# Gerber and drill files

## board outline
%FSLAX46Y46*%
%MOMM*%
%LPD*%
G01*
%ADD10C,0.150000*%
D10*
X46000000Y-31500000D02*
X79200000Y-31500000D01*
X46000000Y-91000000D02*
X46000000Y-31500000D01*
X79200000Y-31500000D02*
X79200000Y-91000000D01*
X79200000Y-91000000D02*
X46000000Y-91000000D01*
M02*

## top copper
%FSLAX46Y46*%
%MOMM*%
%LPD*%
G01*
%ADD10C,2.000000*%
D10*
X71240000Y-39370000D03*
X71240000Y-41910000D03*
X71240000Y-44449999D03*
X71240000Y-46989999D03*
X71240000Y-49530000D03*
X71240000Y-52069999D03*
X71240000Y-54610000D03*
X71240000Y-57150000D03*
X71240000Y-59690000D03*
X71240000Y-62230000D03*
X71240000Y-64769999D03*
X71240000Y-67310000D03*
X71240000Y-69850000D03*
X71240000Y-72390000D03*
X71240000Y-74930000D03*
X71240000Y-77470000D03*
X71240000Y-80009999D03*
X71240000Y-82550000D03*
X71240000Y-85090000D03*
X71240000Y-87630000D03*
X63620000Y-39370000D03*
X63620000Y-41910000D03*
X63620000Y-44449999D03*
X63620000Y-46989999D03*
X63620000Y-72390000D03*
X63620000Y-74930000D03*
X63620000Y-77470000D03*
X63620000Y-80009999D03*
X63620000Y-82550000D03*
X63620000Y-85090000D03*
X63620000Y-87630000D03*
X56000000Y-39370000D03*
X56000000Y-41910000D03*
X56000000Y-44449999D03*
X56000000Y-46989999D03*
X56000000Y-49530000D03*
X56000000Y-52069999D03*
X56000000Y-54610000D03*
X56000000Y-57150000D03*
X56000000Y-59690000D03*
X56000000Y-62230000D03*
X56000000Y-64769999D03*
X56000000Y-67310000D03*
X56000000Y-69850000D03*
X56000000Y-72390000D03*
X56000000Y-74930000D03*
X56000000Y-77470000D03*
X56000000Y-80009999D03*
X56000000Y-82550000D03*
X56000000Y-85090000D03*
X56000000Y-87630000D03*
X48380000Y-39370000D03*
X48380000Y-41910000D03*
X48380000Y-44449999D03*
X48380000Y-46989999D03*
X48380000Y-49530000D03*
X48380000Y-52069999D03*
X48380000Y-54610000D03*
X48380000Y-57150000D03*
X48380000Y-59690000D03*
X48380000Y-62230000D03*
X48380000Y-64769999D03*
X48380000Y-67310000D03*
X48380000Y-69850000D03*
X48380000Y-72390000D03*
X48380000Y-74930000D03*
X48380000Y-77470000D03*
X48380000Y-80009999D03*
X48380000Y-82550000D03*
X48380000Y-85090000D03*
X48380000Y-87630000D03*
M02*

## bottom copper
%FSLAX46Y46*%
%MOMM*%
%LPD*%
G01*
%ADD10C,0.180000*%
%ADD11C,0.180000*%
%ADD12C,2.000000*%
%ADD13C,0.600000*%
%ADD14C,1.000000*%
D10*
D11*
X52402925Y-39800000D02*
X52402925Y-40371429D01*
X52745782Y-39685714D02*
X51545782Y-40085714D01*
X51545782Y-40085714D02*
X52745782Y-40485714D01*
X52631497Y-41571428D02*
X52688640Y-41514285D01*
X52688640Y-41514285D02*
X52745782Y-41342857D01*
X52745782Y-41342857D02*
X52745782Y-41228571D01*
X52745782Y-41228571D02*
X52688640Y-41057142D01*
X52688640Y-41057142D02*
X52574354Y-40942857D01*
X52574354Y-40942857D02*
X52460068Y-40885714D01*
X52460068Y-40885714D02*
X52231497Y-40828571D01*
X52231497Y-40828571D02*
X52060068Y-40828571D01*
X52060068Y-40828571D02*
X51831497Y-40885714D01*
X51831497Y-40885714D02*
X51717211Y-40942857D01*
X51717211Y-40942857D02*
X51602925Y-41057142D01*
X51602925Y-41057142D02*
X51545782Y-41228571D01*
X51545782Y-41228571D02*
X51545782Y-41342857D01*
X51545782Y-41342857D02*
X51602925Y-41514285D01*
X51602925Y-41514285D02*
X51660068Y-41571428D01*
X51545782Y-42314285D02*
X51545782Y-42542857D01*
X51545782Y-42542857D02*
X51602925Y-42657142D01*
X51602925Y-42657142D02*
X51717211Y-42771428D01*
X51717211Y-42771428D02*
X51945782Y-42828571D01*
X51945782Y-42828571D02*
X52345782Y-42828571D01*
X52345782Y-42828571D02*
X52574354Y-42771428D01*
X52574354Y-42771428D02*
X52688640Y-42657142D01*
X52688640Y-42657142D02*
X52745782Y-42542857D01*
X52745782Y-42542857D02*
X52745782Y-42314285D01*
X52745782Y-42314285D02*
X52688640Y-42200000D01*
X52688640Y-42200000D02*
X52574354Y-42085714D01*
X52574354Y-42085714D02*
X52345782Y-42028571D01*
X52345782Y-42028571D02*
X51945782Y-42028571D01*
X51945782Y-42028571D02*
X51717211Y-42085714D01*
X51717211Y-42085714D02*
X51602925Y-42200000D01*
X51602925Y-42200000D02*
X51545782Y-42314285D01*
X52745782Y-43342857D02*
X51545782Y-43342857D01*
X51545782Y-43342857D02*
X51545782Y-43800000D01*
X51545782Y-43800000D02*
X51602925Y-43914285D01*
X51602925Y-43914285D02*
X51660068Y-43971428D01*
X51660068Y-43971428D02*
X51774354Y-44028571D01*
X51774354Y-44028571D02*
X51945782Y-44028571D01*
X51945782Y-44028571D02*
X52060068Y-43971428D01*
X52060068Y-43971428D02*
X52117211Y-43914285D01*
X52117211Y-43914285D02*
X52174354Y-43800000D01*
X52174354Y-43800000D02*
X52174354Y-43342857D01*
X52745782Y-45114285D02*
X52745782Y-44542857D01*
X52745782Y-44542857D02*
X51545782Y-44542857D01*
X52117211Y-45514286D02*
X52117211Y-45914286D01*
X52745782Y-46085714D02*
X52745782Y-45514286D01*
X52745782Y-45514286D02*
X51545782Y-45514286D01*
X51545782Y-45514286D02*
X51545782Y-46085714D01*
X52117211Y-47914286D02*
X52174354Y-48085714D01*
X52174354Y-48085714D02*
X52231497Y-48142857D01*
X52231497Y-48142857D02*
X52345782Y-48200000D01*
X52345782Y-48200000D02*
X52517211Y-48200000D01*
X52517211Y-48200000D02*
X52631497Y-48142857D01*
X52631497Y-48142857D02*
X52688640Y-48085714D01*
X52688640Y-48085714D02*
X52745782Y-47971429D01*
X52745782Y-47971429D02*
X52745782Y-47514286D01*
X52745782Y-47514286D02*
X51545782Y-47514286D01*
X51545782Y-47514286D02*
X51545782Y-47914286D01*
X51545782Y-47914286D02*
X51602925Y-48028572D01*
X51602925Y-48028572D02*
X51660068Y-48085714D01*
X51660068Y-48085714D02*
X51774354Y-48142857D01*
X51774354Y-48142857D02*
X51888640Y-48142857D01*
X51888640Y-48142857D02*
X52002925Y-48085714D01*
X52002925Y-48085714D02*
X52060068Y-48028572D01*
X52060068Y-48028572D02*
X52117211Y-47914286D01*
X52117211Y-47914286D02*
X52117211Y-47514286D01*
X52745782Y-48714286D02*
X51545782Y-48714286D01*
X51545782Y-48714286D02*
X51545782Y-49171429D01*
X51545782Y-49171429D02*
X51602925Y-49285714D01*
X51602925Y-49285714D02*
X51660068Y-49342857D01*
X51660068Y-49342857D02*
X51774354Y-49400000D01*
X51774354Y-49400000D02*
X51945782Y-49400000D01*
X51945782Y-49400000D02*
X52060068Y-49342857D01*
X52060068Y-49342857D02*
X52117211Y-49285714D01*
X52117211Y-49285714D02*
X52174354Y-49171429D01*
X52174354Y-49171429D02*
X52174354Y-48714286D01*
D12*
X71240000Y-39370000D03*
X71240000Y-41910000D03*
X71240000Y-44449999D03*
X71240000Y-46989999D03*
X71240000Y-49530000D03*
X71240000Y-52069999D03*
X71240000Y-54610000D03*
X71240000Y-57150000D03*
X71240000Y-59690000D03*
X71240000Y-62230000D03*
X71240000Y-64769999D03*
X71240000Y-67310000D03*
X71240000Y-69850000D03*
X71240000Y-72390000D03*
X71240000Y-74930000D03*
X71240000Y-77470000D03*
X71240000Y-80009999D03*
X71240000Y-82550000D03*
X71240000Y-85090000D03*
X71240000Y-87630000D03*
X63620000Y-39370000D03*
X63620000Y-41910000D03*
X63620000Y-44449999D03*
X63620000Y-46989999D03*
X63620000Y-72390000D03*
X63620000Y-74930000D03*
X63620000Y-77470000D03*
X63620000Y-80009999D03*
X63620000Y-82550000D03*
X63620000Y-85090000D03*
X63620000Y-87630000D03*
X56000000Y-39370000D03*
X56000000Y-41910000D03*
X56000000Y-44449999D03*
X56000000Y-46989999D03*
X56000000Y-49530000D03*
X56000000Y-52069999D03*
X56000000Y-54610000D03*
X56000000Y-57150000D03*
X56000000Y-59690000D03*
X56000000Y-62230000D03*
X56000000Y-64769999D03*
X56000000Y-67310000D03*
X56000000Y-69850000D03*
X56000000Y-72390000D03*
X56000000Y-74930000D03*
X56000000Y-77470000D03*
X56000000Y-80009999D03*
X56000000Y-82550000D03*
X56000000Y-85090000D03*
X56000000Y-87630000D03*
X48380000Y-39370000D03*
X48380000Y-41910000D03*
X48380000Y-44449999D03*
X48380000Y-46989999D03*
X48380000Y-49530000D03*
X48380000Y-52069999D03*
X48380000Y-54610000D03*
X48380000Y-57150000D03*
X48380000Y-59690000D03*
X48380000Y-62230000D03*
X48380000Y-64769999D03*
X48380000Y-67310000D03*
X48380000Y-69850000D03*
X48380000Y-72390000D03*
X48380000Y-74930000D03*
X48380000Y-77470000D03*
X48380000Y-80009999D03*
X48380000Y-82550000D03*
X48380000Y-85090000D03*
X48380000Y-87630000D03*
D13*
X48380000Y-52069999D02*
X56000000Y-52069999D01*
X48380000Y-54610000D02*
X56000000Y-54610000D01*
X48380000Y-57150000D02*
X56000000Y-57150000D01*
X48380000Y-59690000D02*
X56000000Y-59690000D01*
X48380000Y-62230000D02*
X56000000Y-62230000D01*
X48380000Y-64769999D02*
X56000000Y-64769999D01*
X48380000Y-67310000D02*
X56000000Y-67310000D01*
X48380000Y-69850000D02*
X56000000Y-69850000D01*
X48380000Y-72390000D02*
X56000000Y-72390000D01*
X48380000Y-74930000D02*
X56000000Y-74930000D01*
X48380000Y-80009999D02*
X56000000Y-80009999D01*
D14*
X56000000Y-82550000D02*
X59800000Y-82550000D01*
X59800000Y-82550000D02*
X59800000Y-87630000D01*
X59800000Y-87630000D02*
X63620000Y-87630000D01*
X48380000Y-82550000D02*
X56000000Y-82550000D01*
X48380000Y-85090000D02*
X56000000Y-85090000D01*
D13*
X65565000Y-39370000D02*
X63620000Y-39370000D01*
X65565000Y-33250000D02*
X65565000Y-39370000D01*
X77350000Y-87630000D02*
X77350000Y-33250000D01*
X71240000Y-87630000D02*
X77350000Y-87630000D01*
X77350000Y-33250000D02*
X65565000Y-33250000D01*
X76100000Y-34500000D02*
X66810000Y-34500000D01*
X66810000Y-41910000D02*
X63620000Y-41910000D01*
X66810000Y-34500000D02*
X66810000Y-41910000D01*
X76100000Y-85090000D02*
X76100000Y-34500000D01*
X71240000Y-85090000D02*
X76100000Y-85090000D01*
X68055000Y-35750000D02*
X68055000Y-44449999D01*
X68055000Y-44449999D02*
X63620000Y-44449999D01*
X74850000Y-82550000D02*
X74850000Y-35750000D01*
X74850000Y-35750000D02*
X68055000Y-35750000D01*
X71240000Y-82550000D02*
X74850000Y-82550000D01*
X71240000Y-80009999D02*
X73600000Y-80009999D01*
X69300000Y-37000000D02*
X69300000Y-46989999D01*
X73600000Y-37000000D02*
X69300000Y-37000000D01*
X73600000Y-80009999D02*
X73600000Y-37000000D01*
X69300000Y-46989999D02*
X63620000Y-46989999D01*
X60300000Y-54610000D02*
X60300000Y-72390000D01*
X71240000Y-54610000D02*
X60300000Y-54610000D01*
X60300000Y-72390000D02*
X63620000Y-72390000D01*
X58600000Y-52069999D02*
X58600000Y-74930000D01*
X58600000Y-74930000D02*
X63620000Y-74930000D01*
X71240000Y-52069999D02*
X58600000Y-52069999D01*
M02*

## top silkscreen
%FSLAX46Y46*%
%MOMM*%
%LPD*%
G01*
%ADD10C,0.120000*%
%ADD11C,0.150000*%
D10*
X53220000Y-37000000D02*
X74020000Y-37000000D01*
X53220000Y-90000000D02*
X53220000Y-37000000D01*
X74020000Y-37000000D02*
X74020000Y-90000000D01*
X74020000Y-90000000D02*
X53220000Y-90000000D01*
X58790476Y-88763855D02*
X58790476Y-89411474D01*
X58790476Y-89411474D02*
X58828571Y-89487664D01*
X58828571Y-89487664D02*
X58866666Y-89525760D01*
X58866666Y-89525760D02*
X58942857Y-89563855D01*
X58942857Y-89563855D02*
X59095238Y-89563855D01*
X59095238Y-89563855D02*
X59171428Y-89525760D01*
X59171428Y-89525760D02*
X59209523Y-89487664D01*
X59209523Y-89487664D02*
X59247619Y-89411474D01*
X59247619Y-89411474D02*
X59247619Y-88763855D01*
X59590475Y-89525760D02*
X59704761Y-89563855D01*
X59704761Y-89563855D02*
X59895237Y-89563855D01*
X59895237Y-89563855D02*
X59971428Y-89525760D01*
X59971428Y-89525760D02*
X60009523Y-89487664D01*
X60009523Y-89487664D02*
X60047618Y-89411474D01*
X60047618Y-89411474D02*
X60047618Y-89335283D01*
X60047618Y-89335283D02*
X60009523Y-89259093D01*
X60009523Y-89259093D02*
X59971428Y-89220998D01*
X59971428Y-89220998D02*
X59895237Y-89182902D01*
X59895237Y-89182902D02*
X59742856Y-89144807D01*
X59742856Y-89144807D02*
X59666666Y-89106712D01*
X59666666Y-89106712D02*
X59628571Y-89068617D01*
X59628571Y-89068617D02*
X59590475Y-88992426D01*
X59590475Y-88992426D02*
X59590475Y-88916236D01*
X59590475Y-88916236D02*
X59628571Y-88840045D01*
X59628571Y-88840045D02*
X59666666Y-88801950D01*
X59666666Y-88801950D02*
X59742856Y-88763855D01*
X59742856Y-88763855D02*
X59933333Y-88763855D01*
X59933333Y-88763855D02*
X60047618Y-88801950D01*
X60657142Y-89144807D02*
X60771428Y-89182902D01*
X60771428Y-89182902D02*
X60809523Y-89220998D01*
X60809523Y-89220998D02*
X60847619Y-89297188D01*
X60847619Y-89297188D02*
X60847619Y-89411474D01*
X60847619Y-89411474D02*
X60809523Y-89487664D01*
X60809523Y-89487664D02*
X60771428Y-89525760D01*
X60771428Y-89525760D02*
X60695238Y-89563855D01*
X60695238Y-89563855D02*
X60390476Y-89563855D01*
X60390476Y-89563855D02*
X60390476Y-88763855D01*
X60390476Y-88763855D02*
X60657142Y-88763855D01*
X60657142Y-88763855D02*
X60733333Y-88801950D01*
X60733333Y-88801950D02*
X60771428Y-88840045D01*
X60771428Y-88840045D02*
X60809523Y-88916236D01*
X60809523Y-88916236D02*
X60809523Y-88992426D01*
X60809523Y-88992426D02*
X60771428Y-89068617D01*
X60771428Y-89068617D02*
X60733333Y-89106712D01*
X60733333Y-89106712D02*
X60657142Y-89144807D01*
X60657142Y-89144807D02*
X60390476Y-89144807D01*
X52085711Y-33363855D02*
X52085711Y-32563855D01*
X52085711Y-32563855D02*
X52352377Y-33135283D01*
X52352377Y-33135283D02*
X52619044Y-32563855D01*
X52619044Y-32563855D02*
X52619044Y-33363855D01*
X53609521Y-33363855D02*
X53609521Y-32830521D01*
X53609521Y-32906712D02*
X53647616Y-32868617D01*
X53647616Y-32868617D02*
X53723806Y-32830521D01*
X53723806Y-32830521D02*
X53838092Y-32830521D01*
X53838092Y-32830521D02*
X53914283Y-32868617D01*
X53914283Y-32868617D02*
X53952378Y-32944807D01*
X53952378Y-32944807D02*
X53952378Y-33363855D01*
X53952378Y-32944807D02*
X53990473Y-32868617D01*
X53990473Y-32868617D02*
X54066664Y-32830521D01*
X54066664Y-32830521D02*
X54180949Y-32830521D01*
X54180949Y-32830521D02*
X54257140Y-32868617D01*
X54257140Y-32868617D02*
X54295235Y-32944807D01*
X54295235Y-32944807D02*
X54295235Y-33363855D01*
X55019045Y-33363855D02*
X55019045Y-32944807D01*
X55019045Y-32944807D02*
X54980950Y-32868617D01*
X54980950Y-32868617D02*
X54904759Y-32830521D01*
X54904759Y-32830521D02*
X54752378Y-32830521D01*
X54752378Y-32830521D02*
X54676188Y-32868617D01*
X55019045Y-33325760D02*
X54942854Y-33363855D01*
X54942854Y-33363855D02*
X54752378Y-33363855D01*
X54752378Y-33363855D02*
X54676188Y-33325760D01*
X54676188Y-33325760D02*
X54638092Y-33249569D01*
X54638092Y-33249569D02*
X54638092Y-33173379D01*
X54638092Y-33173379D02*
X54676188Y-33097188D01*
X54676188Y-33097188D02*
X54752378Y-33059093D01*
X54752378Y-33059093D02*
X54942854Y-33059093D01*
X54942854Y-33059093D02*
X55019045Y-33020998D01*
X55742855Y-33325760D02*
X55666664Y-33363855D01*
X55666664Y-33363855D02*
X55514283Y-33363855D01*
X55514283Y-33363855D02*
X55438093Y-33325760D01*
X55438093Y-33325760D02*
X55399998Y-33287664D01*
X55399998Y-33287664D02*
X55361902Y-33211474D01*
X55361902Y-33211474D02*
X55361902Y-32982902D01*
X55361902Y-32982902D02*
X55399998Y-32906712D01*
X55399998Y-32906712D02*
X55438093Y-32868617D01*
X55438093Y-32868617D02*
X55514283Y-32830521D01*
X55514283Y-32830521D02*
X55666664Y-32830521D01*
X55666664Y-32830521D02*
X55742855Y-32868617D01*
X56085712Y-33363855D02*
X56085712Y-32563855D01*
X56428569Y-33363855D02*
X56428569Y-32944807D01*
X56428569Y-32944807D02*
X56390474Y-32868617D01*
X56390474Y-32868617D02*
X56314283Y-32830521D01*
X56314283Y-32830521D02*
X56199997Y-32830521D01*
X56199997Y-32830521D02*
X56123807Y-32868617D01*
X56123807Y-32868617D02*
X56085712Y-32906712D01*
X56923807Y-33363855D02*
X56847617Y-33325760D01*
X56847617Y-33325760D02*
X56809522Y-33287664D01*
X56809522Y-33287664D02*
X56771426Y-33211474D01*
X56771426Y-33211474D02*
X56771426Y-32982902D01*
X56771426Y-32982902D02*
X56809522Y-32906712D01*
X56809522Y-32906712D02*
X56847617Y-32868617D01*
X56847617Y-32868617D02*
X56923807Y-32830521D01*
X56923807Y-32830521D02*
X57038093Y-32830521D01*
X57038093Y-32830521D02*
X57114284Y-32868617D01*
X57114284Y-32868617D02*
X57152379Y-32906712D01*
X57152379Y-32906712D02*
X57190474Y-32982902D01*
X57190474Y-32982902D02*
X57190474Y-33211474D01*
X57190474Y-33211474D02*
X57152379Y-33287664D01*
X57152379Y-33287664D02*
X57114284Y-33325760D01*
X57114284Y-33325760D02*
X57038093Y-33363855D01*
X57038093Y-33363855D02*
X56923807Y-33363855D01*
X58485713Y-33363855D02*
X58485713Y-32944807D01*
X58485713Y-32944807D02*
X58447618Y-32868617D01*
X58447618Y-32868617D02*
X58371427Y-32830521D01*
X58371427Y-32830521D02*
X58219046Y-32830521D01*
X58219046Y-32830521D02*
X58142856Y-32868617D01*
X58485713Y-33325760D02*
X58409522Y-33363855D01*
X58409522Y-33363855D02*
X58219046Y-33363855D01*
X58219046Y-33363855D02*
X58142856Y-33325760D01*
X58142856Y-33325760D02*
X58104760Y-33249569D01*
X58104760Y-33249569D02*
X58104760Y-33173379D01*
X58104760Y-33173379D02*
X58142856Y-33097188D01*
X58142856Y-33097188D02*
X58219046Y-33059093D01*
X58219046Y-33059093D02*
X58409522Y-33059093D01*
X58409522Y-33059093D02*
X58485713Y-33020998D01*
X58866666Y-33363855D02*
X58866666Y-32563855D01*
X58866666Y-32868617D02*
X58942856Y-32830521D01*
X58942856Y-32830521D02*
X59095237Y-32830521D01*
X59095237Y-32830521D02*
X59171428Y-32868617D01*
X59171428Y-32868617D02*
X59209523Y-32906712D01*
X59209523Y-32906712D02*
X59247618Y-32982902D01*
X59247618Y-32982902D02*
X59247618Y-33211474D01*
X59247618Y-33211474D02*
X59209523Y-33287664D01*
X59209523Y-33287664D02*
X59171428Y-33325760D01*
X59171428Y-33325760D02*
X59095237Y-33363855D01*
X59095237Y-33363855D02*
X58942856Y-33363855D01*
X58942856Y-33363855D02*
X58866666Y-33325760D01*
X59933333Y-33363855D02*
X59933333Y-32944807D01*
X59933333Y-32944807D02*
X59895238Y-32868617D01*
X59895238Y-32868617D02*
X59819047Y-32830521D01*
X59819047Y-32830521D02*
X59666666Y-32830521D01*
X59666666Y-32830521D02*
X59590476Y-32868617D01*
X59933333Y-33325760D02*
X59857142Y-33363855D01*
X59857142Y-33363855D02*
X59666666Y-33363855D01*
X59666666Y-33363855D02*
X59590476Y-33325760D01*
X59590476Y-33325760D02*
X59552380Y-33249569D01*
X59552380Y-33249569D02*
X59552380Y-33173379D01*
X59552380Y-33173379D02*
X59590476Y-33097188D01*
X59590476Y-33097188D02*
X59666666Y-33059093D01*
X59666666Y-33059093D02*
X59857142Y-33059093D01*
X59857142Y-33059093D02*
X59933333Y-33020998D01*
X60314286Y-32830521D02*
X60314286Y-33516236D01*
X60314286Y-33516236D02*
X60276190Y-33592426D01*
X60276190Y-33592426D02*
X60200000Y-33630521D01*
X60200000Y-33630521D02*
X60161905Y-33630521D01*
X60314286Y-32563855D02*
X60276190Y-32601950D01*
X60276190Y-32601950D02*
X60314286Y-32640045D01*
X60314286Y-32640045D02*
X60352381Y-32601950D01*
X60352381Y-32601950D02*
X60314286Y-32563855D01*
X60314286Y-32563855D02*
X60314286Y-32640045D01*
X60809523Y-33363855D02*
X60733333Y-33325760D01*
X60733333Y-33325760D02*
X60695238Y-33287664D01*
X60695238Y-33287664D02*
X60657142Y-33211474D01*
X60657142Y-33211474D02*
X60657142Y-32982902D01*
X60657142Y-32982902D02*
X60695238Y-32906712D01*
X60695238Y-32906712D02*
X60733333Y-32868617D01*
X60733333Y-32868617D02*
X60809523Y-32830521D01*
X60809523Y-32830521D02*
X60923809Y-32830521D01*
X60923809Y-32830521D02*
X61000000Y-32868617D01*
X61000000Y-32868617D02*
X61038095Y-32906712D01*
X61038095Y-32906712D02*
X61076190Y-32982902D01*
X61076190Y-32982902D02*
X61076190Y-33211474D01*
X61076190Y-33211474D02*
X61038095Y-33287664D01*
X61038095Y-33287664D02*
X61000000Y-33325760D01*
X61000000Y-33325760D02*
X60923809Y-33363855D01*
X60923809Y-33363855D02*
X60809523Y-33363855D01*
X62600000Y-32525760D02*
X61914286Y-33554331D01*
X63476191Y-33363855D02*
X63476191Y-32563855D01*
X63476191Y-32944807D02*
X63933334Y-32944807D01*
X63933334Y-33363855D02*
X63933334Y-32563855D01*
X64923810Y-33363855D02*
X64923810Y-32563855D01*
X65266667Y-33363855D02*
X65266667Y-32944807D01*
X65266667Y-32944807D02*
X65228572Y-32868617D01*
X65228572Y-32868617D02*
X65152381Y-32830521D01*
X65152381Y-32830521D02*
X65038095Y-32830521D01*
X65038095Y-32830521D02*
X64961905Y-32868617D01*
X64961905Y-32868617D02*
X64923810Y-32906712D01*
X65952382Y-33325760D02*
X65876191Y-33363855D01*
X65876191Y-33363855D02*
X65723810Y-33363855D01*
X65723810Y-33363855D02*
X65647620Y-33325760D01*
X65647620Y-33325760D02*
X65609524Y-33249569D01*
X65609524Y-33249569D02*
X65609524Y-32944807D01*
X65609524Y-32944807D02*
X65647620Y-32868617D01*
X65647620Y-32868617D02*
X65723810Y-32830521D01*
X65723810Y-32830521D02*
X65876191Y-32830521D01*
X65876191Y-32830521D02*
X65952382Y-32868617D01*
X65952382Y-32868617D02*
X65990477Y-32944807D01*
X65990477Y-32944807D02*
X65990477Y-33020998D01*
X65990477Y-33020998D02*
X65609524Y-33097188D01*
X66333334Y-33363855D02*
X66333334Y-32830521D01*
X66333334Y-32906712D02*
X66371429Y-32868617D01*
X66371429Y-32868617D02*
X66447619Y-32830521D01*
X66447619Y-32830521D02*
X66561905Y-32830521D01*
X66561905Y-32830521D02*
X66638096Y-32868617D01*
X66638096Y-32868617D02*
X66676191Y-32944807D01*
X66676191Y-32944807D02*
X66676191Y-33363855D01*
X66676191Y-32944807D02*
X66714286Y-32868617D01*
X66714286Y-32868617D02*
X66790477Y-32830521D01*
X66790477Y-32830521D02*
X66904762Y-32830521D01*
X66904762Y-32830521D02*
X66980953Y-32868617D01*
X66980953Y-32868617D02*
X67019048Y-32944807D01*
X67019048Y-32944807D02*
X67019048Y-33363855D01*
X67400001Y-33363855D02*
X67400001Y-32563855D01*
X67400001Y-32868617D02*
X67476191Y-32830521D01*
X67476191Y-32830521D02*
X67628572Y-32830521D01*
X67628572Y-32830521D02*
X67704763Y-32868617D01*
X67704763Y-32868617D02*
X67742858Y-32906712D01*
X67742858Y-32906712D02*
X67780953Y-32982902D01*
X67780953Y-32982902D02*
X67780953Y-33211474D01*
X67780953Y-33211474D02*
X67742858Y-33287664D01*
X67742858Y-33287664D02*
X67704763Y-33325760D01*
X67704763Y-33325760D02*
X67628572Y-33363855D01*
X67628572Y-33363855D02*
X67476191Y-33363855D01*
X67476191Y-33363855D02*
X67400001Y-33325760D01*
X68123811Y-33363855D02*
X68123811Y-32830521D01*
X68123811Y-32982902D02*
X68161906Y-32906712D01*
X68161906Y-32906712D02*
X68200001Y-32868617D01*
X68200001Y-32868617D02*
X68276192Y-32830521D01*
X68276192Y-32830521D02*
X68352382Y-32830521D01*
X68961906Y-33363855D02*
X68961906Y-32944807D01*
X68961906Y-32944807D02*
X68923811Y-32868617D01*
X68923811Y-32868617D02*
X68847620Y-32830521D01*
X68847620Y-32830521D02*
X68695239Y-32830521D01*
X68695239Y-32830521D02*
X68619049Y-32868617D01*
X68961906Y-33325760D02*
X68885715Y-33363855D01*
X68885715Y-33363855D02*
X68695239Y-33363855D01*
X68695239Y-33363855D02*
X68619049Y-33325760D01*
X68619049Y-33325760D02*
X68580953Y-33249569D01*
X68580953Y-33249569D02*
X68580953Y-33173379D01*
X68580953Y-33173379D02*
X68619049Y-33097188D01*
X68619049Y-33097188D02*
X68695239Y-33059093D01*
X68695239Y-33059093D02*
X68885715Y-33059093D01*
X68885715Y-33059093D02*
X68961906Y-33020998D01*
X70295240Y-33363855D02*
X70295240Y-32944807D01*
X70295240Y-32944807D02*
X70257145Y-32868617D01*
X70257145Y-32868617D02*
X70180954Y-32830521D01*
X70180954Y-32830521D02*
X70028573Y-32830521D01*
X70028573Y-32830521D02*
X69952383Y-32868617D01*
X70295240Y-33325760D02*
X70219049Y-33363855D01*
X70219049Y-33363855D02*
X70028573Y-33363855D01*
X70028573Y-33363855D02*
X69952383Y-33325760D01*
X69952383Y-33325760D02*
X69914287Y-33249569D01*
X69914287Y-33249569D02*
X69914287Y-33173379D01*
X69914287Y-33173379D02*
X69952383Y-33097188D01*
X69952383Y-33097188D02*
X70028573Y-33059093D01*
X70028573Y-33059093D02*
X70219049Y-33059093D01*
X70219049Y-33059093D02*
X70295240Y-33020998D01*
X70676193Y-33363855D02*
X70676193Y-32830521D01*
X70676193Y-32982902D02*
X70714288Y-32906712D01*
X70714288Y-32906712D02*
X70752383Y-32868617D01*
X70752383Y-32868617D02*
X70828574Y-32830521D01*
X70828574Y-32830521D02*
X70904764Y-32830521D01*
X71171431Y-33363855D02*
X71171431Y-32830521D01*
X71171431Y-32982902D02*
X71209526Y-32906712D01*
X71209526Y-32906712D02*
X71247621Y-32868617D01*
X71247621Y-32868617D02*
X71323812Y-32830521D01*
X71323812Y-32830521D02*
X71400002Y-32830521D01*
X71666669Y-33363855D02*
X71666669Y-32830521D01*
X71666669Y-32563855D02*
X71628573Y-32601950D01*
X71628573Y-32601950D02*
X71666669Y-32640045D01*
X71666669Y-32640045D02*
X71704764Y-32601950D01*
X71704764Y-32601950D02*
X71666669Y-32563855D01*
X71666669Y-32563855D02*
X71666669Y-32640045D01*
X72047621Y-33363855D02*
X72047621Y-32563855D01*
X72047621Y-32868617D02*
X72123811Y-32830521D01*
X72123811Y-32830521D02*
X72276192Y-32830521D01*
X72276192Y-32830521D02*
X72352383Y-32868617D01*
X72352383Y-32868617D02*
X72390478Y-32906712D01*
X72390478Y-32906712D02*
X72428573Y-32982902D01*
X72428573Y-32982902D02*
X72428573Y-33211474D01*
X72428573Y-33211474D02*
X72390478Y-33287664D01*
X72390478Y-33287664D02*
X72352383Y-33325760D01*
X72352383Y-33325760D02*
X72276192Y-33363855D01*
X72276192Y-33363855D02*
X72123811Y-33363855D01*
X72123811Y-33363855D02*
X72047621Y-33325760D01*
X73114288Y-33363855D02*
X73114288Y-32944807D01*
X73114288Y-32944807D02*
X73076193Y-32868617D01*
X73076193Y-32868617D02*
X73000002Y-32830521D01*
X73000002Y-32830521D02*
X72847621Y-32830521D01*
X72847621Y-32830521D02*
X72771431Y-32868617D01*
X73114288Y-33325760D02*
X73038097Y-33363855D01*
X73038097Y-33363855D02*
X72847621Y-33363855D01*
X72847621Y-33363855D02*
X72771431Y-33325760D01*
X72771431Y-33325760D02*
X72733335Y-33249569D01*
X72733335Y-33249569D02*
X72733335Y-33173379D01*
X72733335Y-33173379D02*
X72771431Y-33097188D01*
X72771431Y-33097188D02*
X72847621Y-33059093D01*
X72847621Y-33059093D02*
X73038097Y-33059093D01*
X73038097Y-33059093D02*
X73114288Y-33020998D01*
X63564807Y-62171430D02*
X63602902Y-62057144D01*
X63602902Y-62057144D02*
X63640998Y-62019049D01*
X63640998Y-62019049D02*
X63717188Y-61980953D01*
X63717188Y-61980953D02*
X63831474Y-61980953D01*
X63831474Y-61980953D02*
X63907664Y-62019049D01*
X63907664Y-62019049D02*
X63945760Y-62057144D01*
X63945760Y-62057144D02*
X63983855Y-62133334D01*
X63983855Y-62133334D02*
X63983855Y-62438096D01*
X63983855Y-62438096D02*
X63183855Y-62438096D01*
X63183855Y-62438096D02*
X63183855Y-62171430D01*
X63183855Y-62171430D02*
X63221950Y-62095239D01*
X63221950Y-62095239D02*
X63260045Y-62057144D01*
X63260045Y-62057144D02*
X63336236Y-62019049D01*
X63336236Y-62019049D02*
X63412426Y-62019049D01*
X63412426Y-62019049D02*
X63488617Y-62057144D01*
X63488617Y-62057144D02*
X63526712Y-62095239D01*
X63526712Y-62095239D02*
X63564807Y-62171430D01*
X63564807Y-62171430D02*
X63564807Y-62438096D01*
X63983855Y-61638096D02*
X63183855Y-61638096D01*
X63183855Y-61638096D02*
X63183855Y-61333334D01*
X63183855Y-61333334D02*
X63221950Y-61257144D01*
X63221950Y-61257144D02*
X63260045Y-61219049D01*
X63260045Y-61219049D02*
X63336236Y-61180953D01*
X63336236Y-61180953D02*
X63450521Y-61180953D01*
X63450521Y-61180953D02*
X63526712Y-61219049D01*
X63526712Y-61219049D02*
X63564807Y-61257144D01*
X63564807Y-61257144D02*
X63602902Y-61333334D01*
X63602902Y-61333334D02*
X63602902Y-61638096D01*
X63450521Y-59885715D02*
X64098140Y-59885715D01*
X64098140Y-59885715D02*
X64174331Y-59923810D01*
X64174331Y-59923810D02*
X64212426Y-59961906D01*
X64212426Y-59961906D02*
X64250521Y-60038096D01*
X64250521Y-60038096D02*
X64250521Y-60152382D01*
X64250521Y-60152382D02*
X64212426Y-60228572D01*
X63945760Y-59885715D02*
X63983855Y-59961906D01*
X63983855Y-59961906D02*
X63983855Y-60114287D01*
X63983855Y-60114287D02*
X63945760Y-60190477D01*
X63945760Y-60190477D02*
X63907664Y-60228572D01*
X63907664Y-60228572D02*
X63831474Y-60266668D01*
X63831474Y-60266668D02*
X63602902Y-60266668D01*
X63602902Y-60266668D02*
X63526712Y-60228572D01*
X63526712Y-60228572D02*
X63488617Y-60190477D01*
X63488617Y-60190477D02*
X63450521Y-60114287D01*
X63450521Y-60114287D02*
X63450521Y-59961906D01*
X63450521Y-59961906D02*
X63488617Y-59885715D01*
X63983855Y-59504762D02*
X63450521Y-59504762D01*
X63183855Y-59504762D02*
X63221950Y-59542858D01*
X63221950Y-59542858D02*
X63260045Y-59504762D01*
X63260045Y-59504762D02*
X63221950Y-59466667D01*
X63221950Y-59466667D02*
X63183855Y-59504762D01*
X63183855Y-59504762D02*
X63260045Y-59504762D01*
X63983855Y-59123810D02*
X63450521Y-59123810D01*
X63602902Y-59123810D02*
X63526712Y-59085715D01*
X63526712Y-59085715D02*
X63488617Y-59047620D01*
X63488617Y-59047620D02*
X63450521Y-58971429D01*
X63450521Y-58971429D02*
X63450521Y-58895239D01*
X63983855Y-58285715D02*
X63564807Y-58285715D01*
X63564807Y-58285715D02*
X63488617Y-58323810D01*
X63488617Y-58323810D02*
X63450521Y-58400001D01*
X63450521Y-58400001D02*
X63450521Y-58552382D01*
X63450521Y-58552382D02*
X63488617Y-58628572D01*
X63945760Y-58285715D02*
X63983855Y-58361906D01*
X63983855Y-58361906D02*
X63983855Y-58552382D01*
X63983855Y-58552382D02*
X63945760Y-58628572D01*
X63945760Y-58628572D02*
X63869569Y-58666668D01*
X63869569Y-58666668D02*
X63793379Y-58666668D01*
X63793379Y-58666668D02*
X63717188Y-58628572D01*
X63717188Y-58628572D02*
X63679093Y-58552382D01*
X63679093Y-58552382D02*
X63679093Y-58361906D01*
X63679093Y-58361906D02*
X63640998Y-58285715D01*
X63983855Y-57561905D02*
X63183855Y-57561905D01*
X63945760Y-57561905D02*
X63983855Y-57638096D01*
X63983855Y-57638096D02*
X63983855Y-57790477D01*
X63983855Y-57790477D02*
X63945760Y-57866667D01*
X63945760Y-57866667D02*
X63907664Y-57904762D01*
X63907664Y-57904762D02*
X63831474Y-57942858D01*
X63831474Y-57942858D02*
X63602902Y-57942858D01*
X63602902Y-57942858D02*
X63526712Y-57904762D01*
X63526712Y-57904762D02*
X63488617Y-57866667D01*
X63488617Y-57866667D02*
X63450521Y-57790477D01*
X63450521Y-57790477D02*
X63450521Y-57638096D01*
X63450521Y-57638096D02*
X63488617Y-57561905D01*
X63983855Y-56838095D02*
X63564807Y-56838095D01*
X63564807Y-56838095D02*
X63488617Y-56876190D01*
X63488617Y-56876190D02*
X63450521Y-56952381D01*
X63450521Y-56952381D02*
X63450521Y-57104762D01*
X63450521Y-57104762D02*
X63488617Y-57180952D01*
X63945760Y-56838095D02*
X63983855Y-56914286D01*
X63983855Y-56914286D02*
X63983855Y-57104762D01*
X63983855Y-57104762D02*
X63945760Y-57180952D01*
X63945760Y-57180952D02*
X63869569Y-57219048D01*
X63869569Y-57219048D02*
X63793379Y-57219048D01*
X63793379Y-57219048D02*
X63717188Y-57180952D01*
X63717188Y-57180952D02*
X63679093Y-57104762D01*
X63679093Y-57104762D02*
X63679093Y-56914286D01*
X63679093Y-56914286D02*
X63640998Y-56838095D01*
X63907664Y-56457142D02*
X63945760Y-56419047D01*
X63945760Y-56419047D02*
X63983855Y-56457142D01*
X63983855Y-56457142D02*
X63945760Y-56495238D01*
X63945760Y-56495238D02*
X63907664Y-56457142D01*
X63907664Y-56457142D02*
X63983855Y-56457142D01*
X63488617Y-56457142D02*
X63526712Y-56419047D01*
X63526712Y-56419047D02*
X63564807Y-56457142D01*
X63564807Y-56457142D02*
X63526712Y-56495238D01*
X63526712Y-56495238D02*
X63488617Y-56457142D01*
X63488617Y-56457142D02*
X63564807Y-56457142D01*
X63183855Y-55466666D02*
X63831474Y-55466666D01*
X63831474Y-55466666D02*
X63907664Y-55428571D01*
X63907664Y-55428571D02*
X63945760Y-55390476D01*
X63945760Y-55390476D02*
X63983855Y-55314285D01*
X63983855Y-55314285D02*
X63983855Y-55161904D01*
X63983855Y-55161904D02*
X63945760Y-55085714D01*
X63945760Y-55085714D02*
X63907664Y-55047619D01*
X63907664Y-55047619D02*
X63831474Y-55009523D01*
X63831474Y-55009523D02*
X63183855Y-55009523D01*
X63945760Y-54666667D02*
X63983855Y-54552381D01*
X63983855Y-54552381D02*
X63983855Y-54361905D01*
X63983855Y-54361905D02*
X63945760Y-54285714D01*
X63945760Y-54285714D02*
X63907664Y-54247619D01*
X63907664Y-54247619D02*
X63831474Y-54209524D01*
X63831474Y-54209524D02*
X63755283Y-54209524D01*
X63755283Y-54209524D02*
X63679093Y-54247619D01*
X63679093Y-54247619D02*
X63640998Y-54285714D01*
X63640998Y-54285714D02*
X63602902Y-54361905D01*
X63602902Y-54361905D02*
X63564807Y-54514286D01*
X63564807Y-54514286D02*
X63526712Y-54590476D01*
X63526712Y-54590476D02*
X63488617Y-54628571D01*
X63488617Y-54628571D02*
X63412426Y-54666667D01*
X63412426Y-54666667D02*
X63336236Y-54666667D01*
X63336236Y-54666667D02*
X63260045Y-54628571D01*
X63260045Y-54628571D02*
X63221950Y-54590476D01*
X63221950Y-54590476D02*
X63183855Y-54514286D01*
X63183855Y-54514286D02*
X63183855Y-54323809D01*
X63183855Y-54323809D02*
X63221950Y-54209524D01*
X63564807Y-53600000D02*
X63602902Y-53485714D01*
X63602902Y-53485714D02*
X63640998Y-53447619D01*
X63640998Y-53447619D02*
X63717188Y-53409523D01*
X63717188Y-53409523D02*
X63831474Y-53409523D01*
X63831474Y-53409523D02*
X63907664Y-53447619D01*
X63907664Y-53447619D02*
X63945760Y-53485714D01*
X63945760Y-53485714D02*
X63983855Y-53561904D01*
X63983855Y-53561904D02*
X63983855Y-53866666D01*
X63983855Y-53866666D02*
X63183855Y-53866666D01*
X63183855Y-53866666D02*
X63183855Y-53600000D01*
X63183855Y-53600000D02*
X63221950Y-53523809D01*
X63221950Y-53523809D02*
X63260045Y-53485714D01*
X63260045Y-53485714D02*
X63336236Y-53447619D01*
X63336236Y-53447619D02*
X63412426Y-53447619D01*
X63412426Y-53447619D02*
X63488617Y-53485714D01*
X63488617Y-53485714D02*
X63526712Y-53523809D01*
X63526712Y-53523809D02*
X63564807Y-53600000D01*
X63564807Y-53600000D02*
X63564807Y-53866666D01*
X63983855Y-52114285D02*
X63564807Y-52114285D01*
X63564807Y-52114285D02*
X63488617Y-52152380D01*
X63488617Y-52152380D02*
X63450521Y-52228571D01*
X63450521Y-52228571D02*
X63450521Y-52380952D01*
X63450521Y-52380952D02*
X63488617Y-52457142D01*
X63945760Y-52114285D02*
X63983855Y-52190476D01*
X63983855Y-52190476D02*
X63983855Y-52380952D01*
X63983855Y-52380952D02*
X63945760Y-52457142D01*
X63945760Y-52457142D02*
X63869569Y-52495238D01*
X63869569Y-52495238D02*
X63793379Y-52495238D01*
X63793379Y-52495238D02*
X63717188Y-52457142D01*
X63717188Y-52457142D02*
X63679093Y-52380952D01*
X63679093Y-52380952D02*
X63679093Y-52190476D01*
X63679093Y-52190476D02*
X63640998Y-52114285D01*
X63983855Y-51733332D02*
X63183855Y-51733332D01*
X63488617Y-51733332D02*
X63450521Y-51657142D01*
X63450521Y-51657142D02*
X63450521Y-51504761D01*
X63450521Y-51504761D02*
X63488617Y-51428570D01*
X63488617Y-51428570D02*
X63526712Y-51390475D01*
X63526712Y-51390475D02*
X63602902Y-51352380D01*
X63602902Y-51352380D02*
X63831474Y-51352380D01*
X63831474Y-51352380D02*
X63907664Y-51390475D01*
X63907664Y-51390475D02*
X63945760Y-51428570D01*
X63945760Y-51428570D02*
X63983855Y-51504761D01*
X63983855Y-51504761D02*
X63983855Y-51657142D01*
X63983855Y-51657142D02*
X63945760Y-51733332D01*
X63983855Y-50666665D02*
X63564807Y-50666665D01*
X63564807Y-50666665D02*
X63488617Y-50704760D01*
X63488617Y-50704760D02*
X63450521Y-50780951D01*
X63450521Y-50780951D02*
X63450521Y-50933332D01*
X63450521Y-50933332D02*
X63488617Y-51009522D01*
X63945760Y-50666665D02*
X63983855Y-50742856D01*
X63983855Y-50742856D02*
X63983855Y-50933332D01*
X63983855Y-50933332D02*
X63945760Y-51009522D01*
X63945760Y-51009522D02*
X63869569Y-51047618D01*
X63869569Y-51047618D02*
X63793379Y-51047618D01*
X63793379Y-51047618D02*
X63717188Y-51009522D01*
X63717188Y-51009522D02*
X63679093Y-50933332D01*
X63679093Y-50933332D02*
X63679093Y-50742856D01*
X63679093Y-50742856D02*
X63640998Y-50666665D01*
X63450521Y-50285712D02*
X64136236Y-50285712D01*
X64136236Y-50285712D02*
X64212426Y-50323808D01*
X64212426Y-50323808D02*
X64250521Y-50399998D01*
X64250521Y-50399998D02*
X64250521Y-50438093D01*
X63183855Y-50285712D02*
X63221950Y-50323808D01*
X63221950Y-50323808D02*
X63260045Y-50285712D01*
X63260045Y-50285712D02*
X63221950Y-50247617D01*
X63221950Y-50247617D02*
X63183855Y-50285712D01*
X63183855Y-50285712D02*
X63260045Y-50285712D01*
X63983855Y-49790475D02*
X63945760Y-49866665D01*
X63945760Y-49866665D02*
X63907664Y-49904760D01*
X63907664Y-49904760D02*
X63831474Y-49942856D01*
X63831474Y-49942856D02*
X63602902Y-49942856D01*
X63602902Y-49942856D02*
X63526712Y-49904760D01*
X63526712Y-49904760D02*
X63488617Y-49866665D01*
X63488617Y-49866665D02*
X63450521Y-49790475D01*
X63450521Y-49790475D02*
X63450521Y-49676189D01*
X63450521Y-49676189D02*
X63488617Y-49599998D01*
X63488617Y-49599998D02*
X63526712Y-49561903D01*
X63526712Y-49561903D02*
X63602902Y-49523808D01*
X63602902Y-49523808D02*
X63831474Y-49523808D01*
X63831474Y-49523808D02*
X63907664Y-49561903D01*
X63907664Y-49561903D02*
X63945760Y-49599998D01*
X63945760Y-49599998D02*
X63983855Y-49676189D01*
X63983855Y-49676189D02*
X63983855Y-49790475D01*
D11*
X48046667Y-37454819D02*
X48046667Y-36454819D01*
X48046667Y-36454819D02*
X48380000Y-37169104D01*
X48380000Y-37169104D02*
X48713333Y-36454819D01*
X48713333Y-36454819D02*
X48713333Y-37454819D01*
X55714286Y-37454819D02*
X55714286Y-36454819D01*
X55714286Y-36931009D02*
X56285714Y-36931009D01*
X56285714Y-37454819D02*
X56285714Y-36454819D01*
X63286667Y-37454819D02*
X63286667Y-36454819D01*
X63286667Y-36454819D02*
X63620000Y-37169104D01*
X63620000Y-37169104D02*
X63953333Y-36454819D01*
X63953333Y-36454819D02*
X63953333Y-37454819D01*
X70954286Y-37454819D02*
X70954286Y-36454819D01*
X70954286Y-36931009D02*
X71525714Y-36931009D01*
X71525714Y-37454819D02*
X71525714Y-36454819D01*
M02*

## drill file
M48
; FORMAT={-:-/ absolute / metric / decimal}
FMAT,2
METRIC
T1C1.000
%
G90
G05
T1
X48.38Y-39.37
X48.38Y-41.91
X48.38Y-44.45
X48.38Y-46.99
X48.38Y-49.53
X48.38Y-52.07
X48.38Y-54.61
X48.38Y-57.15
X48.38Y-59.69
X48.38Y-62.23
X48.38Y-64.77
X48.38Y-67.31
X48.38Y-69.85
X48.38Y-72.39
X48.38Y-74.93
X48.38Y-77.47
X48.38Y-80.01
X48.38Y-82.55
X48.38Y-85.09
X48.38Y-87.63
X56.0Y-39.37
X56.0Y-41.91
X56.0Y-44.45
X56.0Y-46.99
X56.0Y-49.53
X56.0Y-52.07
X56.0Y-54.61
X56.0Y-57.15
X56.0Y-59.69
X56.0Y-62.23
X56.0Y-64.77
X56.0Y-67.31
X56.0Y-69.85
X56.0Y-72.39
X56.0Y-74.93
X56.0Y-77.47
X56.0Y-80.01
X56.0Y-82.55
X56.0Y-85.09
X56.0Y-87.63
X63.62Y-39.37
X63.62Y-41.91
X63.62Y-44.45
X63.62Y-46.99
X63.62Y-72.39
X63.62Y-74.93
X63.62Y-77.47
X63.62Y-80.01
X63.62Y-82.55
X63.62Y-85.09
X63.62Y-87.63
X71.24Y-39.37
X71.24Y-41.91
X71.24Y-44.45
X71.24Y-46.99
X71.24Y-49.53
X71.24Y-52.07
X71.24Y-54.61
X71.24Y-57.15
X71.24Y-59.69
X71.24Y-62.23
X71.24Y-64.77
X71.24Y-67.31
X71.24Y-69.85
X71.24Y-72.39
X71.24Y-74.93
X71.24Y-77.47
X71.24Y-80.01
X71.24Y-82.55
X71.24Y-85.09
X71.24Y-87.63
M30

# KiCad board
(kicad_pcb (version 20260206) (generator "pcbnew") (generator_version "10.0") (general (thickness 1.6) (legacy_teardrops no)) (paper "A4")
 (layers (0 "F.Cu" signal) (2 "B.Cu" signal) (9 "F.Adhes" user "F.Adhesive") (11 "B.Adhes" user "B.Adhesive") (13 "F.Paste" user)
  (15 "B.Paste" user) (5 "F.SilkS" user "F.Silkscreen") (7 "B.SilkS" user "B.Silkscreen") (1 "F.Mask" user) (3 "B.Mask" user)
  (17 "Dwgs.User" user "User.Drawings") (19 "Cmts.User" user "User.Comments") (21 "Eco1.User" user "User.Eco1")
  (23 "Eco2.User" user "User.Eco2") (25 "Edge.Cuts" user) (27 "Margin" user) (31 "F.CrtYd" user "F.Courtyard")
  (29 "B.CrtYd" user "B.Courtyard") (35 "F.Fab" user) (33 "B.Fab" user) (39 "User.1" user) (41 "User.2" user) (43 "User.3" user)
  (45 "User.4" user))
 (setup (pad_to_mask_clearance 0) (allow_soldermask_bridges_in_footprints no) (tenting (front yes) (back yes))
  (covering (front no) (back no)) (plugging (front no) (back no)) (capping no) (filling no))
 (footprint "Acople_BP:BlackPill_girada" (layer "F.Cu") (at 63.62 63.5)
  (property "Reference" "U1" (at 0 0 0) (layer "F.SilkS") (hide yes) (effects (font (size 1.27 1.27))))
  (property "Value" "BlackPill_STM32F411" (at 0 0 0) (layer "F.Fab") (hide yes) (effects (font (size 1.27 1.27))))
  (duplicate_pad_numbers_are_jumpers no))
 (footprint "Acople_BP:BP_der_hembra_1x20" (layer "F.Cu") (at 71.24 63.5)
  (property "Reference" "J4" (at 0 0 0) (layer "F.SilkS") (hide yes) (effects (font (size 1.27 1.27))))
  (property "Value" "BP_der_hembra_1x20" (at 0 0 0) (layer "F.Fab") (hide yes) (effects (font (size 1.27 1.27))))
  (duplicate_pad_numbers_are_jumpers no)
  (pad "1" thru_hole circle (at 0 -24.13) (size 2 2) (drill 1) (layers "*.Cu" "*.Mask") (remove_unused_layers no))
  (pad "2" thru_hole circle (at 0 -21.59) (size 2 2) (drill 1) (layers "*.Cu" "*.Mask") (remove_unused_layers no))
  (pad "3" thru_hole circle (at 0 -19.050001) (size 2 2) (drill 1) (layers "*.Cu" "*.Mask") (remove_unused_layers no))
  (pad "4" thru_hole circle (at 0 -16.510001) (size 2 2) (drill 1) (layers "*.Cu" "*.Mask") (remove_unused_layers no))
  (pad "5" thru_hole circle (at 0 -13.97) (size 2 2) (drill 1) (layers "*.Cu" "*.Mask") (remove_unused_layers no))
  (pad "6" thru_hole circle (at 0 -11.430001) (size 2 2) (drill 1) (layers "*.Cu" "*.Mask") (remove_unused_layers no) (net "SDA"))
  (pad "7" thru_hole circle (at 0 -8.89) (size 2 2) (drill 1) (layers "*.Cu" "*.Mask") (remove_unused_layers no) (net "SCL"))
  (pad "8" thru_hole circle (at 0 -6.35) (size 2 2) (drill 1) (layers "*.Cu" "*.Mask") (remove_unused_layers no))
  (pad "9" thru_hole circle (at 0 -3.81) (size 2 2) (drill 1) (layers "*.Cu" "*.Mask") (remove_unused_layers no))
  (pad "10" thru_hole circle (at 0 -1.27) (size 2 2) (drill 1) (layers "*.Cu" "*.Mask") (remove_unused_layers no))
  (pad "11" thru_hole circle (at 0 1.269999) (size 2 2) (drill 1) (layers "*.Cu" "*.Mask") (remove_unused_layers no))
  (pad "12" thru_hole circle (at 0 3.81) (size 2 2) (drill 1) (layers "*.Cu" "*.Mask") (remove_unused_layers no))
  (pad "13" thru_hole circle (at 0 6.35) (size 2 2) (drill 1) (layers "*.Cu" "*.Mask") (remove_unused_layers no))
  (pad "14" thru_hole circle (at 0 8.89) (size 2 2) (drill 1) (layers "*.Cu" "*.Mask") (remove_unused_layers no))
  (pad "15" thru_hole circle (at 0 11.43) (size 2 2) (drill 1) (layers "*.Cu" "*.Mask") (remove_unused_layers no))
  (pad "16" thru_hole circle (at 0 13.97) (size 2 2) (drill 1) (layers "*.Cu" "*.Mask") (remove_unused_layers no))
  (pad "17" thru_hole circle (at 0 16.509999) (size 2 2) (drill 1) (layers "*.Cu" "*.Mask") (remove_unused_layers no) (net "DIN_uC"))
  (pad "18" thru_hole circle (at 0 19.05) (size 2 2) (drill 1) (layers "*.Cu" "*.Mask") (remove_unused_layers no) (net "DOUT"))
  (pad "19" thru_hole circle (at 0 21.59) (size 2 2) (drill 1) (layers "*.Cu" "*.Mask") (remove_unused_layers no) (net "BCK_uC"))
  (pad "20" thru_hole circle (at 0 24.13) (size 2 2) (drill 1) (layers "*.Cu" "*.Mask") (remove_unused_layers no) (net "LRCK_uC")))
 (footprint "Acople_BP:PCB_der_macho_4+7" (layer "F.Cu") (at 63.62 63.5)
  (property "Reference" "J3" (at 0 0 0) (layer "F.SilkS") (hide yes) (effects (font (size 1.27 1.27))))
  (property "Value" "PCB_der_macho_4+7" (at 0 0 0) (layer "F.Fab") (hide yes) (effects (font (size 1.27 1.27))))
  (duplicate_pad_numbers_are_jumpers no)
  (pad "1" thru_hole circle (at 0 -24.13) (size 2 2) (drill 1) (layers "*.Cu" "*.Mask") (remove_unused_layers no) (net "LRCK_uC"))
  (pad "2" thru_hole circle (at 0 -21.59) (size 2 2) (drill 1) (layers "*.Cu" "*.Mask") (remove_unused_layers no) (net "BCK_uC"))
  (pad "3" thru_hole circle (at 0 -19.050001) (size 2 2) (drill 1) (layers "*.Cu" "*.Mask") (remove_unused_layers no) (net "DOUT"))
  (pad "4" thru_hole circle (at 0 -16.510001) (size 2 2) (drill 1) (layers "*.Cu" "*.Mask") (remove_unused_layers no) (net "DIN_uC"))
  (pad "14" thru_hole circle (at 0 8.89) (size 2 2) (drill 1) (layers "*.Cu" "*.Mask") (remove_unused_layers no) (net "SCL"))
  (pad "15" thru_hole circle (at 0 11.43) (size 2 2) (drill 1) (layers "*.Cu" "*.Mask") (remove_unused_layers no) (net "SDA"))
  (pad "16" thru_hole circle (at 0 13.97) (size 2 2) (drill 1) (layers "*.Cu" "*.Mask") (remove_unused_layers no))
  (pad "17" thru_hole circle (at 0 16.509999) (size 2 2) (drill 1) (layers "*.Cu" "*.Mask") (remove_unused_layers no))
  (pad "18" thru_hole circle (at 0 19.05) (size 2 2) (drill 1) (layers "*.Cu" "*.Mask") (remove_unused_layers no))
  (pad "19" thru_hole circle (at 0 21.59) (size 2 2) (drill 1) (layers "*.Cu" "*.Mask") (remove_unused_layers no))
  (pad "20" thru_hole circle (at 0 24.13) (size 2 2) (drill 1) (layers "*.Cu" "*.Mask") (remove_unused_layers no) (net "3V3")))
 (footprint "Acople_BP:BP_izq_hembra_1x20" (layer "F.Cu") (at 56 63.5)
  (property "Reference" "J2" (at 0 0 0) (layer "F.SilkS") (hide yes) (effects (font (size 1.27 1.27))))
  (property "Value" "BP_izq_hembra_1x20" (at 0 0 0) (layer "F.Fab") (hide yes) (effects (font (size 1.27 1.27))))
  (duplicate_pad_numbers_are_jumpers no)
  (pad "1" thru_hole circle (at 0 -24.13) (size 2 2) (drill 1) (layers "*.Cu" "*.Mask") (remove_unused_layers no))
  (pad "2" thru_hole circle (at 0 -21.59) (size 2 2) (drill 1) (layers "*.Cu" "*.Mask") (remove_unused_layers no))
  (pad "3" thru_hole circle (at 0 -19.050001) (size 2 2) (drill 1) (layers "*.Cu" "*.Mask") (remove_unused_layers no))
  (pad "4" thru_hole circle (at 0 -16.510001) (size 2 2) (drill 1) (layers "*.Cu" "*.Mask") (remove_unused_layers no))
  (pad "5" thru_hole circle (at 0 -13.97) (size 2 2) (drill 1) (layers "*.Cu" "*.Mask") (remove_unused_layers no))
  (pad "6" thru_hole circle (at 0 -11.430001) (size 2 2) (drill 1) (layers "*.Cu" "*.Mask") (remove_unused_layers no) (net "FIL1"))
  (pad "7" thru_hole circle (at 0 -8.89) (size 2 2) (drill 1) (layers "*.Cu" "*.Mask") (remove_unused_layers no) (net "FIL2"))
  (pad "8" thru_hole circle (at 0 -6.35) (size 2 2) (drill 1) (layers "*.Cu" "*.Mask") (remove_unused_layers no) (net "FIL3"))
  (pad "9" thru_hole circle (at 0 -3.81) (size 2 2) (drill 1) (layers "*.Cu" "*.Mask") (remove_unused_layers no) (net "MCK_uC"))
  (pad "10" thru_hole circle (at 0 -1.27) (size 2 2) (drill 1) (layers "*.Cu" "*.Mask") (remove_unused_layers no) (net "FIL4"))
  (pad "11" thru_hole circle (at 0 1.269999) (size 2 2) (drill 1) (layers "*.Cu" "*.Mask") (remove_unused_layers no) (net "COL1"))
  (pad "12" thru_hole circle (at 0 3.81) (size 2 2) (drill 1) (layers "*.Cu" "*.Mask") (remove_unused_layers no) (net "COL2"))
  (pad "13" thru_hole circle (at 0 6.35) (size 2 2) (drill 1) (layers "*.Cu" "*.Mask") (remove_unused_layers no) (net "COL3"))
  (pad "14" thru_hole circle (at 0 8.89) (size 2 2) (drill 1) (layers "*.Cu" "*.Mask") (remove_unused_layers no) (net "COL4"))
  (pad "15" thru_hole circle (at 0 11.43) (size 2 2) (drill 1) (layers "*.Cu" "*.Mask") (remove_unused_layers no) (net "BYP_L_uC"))
  (pad "16" thru_hole circle (at 0 13.97) (size 2 2) (drill 1) (layers "*.Cu" "*.Mask") (remove_unused_layers no))
  (pad "17" thru_hole circle (at 0 16.509999) (size 2 2) (drill 1) (layers "*.Cu" "*.Mask") (remove_unused_layers no) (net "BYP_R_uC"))
  (pad "18" thru_hole circle (at 0 19.05) (size 2 2) (drill 1) (layers "*.Cu" "*.Mask") (remove_unused_layers no) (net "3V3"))
  (pad "19" thru_hole circle (at 0 21.59) (size 2 2) (drill 1) (layers "*.Cu" "*.Mask") (remove_unused_layers no) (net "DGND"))
  (pad "20" thru_hole circle (at 0 24.13) (size 2 2) (drill 1) (layers "*.Cu" "*.Mask") (remove_unused_layers no)))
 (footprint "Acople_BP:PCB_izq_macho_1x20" (layer "F.Cu") (at 48.38 63.5)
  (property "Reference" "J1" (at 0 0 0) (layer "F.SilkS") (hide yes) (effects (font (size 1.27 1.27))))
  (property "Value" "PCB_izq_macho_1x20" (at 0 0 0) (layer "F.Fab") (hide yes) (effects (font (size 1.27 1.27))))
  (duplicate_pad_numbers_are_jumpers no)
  (pad "1" thru_hole circle (at 0 -24.13) (size 2 2) (drill 1) (layers "*.Cu" "*.Mask") (remove_unused_layers no))
  (pad "2" thru_hole circle (at 0 -21.59) (size 2 2) (drill 1) (layers "*.Cu" "*.Mask") (remove_unused_layers no))
  (pad "3" thru_hole circle (at 0 -19.050001) (size 2 2) (drill 1) (layers "*.Cu" "*.Mask") (remove_unused_layers no))
  (pad "4" thru_hole circle (at 0 -16.510001) (size 2 2) (drill 1) (layers "*.Cu" "*.Mask") (remove_unused_layers no))
  (pad "5" thru_hole circle (at 0 -13.97) (size 2 2) (drill 1) (layers "*.Cu" "*.Mask") (remove_unused_layers no))
  (pad "6" thru_hole circle (at 0 -11.430001) (size 2 2) (drill 1) (layers "*.Cu" "*.Mask") (remove_unused_layers no) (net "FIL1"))
  (pad "7" thru_hole circle (at 0 -8.89) (size 2 2) (drill 1) (layers "*.Cu" "*.Mask") (remove_unused_layers no) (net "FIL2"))
  (pad "8" thru_hole circle (at 0 -6.35) (size 2 2) (drill 1) (layers "*.Cu" "*.Mask") (remove_unused_layers no) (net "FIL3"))
  (pad "9" thru_hole circle (at 0 -3.81) (size 2 2) (drill 1) (layers "*.Cu" "*.Mask") (remove_unused_layers no) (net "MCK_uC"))
  (pad "10" thru_hole circle (at 0 -1.27) (size 2 2) (drill 1) (layers "*.Cu" "*.Mask") (remove_unused_layers no) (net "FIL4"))
  (pad "11" thru_hole circle (at 0 1.269999) (size 2 2) (drill 1) (layers "*.Cu" "*.Mask") (remove_unused_layers no) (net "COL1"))
  (pad "12" thru_hole circle (at 0 3.81) (size 2 2) (drill 1) (layers "*.Cu" "*.Mask") (remove_unused_layers no) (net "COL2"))
  (pad "13" thru_hole circle (at 0 6.35) (size 2 2) (drill 1) (layers "*.Cu" "*.Mask") (remove_unused_layers no) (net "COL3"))
  (pad "14" thru_hole circle (at 0 8.89) (size 2 2) (drill 1) (layers "*.Cu" "*.Mask") (remove_unused_layers no) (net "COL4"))
  (pad "15" thru_hole circle (at 0 11.43) (size 2 2) (drill 1) (layers "*.Cu" "*.Mask") (remove_unused_layers no) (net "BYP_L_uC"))
  (pad "16" thru_hole circle (at 0 13.97) (size 2 2) (drill 1) (layers "*.Cu" "*.Mask") (remove_unused_layers no))
  (pad "17" thru_hole circle (at 0 16.509999) (size 2 2) (drill 1) (layers "*.Cu" "*.Mask") (remove_unused_layers no) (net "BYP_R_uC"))
  (pad "18" thru_hole circle (at 0 19.05) (size 2 2) (drill 1) (layers "*.Cu" "*.Mask") (remove_unused_layers no) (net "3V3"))
  (pad "19" thru_hole circle (at 0 21.59) (size 2 2) (drill 1) (layers "*.Cu" "*.Mask") (remove_unused_layers no) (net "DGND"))
  (pad "20" thru_hole circle (at 0 24.13) (size 2 2) (drill 1) (layers "*.Cu" "*.Mask") (remove_unused_layers no)))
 (gr_line (start 53.22 37) (end 74.02 37) (stroke (width 0.12) (type default)) (layer "F.SilkS"))
 (gr_line (start 53.22 90) (end 53.22 37) (stroke (width 0.12) (type default)) (layer "F.SilkS"))
 (gr_line (start 74.02 37) (end 74.02 90) (stroke (width 0.12) (type default)) (layer "F.SilkS"))
 (gr_line (start 74.02 90) (end 53.22 90) (stroke (width 0.12) (type default)) (layer "F.SilkS"))
 (gr_line (start 46 31.5) (end 79.2 31.5) (stroke (width 0.15) (type default)) (layer "Edge.Cuts"))
 (gr_line (start 46 91) (end 46 31.5) (stroke (width 0.15) (type default)) (layer "Edge.Cuts"))
 (gr_line (start 79.2 31.5) (end 79.2 91) (stroke (width 0.15) (type default)) (layer "Edge.Cuts"))
 (gr_line (start 79.2 91) (end 46 91) (stroke (width 0.15) (type default)) (layer "Edge.Cuts"))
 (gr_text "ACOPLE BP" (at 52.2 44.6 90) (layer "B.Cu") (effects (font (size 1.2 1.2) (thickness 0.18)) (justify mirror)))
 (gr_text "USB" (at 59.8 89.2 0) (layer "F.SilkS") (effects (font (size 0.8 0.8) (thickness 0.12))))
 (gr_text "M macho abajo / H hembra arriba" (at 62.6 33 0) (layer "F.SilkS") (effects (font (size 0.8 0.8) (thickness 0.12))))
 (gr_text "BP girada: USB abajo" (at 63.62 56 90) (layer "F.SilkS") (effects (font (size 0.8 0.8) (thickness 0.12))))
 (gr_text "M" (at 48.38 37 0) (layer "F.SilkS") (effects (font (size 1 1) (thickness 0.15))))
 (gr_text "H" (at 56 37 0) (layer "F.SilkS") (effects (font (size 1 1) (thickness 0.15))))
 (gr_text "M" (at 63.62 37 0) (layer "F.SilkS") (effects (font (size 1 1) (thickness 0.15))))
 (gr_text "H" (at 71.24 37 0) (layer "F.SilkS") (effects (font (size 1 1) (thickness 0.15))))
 (segment (start 48.38 52.069999) (end 56 52.069999) (width 0.6) (layer "B.Cu") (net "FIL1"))
 (segment (start 48.38 54.61) (end 56 54.61) (width 0.6) (layer "B.Cu") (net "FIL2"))
 (segment (start 48.38 57.15) (end 56 57.15) (width 0.6) (layer "B.Cu") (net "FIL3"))
 (segment (start 48.38 59.69) (end 56 59.69) (width 0.6) (layer "B.Cu") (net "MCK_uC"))
 (segment (start 48.38 62.23) (end 56 62.23) (width 0.6) (layer "B.Cu") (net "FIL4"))
 (segment (start 48.38 64.769999) (end 56 64.769999) (width 0.6) (layer "B.Cu") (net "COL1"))
 (segment (start 48.38 67.31) (end 56 67.31) (width 0.6) (layer "B.Cu") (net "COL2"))
 (segment (start 48.38 69.85) (end 56 69.85) (width 0.6) (layer "B.Cu") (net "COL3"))
 (segment (start 48.38 72.39) (end 56 72.39) (width 0.6) (layer "B.Cu") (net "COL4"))
 (segment (start 48.38 74.93) (end 56 74.93) (width 0.6) (layer "B.Cu") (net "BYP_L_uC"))
 (segment (start 48.38 80.009999) (end 56 80.009999) (width 0.6) (layer "B.Cu") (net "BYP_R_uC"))
 (segment (start 56 82.55) (end 59.8 82.55) (width 1) (layer "B.Cu") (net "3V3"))
 (segment (start 59.8 82.55) (end 59.8 87.63) (width 1) (layer "B.Cu") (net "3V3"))
 (segment (start 59.8 87.63) (end 63.62 87.63) (width 1) (layer "B.Cu") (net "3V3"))
 (segment (start 48.38 82.55) (end 56 82.55) (width 1) (layer "B.Cu") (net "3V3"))
 (segment (start 48.38 85.09) (end 56 85.09) (width 1) (layer "B.Cu") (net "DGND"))
 (segment (start 65.565 39.37) (end 63.62 39.37) (width 0.6) (layer "B.Cu") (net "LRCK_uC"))
 (segment (start 65.565 33.25) (end 65.565 39.37) (width 0.6) (layer "B.Cu") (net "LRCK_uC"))
 (segment (start 77.35 87.63) (end 77.35 33.25) (width 0.6) (layer "B.Cu") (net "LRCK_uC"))
 (segment (start 71.24 87.63) (end 77.35 87.63) (width 0.6) (layer "B.Cu") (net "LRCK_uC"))
 (segment (start 77.35 33.25) (end 65.565 33.25) (width 0.6) (layer "B.Cu") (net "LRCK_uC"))
 (segment (start 76.1 34.5) (end 66.81 34.5) (width 0.6) (layer "B.Cu") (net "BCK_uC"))
 (segment (start 66.81 41.91) (end 63.62 41.91) (width 0.6) (layer "B.Cu") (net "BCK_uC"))
 (segment (start 66.81 34.5) (end 66.81 41.91) (width 0.6) (layer "B.Cu") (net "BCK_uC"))
 (segment (start 76.1 85.09) (end 76.1 34.5) (width 0.6) (layer "B.Cu") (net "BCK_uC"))
 (segment (start 71.24 85.09) (end 76.1 85.09) (width 0.6) (layer "B.Cu") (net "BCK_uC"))
 (segment (start 68.055 35.75) (end 68.055 44.449999) (width 0.6) (layer "B.Cu") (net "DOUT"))
 (segment (start 68.055 44.449999) (end 63.62 44.449999) (width 0.6) (layer "B.Cu") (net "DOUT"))
 (segment (start 74.85 82.55) (end 74.85 35.75) (width 0.6) (layer "B.Cu") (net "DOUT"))
 (segment (start 74.85 35.75) (end 68.055 35.75) (width 0.6) (layer "B.Cu") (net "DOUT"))
 (segment (start 71.24 82.55) (end 74.85 82.55) (width 0.6) (layer "B.Cu") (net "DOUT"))
 (segment (start 71.24 80.009999) (end 73.6 80.009999) (width 0.6) (layer "B.Cu") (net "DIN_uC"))
 (segment (start 69.3 37) (end 69.3 46.989999) (width 0.6) (layer "B.Cu") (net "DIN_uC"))
 (segment (start 73.6 37) (end 69.3 37) (width 0.6) (layer "B.Cu") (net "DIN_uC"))
 (segment (start 73.6 80.009999) (end 73.6 37) (width 0.6) (layer "B.Cu") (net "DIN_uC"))
 (segment (start 69.3 46.989999) (end 63.62 46.989999) (width 0.6) (layer "B.Cu") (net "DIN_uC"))
 (segment (start 60.3 54.61) (end 60.3 72.39) (width 0.6) (layer "B.Cu") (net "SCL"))
 (segment (start 71.24 54.61) (end 60.3 54.61) (width 0.6) (layer "B.Cu") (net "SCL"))
 (segment (start 60.3 72.39) (end 63.62 72.39) (width 0.6) (layer "B.Cu") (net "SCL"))
 (segment (start 58.6 52.069999) (end 58.6 74.93) (width 0.6) (layer "B.Cu") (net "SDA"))
 (segment (start 58.6 74.93) (end 63.62 74.93) (width 0.6) (layer "B.Cu") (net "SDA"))
 (segment (start 71.24 52.069999) (end 58.6 52.069999) (width 0.6) (layer "B.Cu") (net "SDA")))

